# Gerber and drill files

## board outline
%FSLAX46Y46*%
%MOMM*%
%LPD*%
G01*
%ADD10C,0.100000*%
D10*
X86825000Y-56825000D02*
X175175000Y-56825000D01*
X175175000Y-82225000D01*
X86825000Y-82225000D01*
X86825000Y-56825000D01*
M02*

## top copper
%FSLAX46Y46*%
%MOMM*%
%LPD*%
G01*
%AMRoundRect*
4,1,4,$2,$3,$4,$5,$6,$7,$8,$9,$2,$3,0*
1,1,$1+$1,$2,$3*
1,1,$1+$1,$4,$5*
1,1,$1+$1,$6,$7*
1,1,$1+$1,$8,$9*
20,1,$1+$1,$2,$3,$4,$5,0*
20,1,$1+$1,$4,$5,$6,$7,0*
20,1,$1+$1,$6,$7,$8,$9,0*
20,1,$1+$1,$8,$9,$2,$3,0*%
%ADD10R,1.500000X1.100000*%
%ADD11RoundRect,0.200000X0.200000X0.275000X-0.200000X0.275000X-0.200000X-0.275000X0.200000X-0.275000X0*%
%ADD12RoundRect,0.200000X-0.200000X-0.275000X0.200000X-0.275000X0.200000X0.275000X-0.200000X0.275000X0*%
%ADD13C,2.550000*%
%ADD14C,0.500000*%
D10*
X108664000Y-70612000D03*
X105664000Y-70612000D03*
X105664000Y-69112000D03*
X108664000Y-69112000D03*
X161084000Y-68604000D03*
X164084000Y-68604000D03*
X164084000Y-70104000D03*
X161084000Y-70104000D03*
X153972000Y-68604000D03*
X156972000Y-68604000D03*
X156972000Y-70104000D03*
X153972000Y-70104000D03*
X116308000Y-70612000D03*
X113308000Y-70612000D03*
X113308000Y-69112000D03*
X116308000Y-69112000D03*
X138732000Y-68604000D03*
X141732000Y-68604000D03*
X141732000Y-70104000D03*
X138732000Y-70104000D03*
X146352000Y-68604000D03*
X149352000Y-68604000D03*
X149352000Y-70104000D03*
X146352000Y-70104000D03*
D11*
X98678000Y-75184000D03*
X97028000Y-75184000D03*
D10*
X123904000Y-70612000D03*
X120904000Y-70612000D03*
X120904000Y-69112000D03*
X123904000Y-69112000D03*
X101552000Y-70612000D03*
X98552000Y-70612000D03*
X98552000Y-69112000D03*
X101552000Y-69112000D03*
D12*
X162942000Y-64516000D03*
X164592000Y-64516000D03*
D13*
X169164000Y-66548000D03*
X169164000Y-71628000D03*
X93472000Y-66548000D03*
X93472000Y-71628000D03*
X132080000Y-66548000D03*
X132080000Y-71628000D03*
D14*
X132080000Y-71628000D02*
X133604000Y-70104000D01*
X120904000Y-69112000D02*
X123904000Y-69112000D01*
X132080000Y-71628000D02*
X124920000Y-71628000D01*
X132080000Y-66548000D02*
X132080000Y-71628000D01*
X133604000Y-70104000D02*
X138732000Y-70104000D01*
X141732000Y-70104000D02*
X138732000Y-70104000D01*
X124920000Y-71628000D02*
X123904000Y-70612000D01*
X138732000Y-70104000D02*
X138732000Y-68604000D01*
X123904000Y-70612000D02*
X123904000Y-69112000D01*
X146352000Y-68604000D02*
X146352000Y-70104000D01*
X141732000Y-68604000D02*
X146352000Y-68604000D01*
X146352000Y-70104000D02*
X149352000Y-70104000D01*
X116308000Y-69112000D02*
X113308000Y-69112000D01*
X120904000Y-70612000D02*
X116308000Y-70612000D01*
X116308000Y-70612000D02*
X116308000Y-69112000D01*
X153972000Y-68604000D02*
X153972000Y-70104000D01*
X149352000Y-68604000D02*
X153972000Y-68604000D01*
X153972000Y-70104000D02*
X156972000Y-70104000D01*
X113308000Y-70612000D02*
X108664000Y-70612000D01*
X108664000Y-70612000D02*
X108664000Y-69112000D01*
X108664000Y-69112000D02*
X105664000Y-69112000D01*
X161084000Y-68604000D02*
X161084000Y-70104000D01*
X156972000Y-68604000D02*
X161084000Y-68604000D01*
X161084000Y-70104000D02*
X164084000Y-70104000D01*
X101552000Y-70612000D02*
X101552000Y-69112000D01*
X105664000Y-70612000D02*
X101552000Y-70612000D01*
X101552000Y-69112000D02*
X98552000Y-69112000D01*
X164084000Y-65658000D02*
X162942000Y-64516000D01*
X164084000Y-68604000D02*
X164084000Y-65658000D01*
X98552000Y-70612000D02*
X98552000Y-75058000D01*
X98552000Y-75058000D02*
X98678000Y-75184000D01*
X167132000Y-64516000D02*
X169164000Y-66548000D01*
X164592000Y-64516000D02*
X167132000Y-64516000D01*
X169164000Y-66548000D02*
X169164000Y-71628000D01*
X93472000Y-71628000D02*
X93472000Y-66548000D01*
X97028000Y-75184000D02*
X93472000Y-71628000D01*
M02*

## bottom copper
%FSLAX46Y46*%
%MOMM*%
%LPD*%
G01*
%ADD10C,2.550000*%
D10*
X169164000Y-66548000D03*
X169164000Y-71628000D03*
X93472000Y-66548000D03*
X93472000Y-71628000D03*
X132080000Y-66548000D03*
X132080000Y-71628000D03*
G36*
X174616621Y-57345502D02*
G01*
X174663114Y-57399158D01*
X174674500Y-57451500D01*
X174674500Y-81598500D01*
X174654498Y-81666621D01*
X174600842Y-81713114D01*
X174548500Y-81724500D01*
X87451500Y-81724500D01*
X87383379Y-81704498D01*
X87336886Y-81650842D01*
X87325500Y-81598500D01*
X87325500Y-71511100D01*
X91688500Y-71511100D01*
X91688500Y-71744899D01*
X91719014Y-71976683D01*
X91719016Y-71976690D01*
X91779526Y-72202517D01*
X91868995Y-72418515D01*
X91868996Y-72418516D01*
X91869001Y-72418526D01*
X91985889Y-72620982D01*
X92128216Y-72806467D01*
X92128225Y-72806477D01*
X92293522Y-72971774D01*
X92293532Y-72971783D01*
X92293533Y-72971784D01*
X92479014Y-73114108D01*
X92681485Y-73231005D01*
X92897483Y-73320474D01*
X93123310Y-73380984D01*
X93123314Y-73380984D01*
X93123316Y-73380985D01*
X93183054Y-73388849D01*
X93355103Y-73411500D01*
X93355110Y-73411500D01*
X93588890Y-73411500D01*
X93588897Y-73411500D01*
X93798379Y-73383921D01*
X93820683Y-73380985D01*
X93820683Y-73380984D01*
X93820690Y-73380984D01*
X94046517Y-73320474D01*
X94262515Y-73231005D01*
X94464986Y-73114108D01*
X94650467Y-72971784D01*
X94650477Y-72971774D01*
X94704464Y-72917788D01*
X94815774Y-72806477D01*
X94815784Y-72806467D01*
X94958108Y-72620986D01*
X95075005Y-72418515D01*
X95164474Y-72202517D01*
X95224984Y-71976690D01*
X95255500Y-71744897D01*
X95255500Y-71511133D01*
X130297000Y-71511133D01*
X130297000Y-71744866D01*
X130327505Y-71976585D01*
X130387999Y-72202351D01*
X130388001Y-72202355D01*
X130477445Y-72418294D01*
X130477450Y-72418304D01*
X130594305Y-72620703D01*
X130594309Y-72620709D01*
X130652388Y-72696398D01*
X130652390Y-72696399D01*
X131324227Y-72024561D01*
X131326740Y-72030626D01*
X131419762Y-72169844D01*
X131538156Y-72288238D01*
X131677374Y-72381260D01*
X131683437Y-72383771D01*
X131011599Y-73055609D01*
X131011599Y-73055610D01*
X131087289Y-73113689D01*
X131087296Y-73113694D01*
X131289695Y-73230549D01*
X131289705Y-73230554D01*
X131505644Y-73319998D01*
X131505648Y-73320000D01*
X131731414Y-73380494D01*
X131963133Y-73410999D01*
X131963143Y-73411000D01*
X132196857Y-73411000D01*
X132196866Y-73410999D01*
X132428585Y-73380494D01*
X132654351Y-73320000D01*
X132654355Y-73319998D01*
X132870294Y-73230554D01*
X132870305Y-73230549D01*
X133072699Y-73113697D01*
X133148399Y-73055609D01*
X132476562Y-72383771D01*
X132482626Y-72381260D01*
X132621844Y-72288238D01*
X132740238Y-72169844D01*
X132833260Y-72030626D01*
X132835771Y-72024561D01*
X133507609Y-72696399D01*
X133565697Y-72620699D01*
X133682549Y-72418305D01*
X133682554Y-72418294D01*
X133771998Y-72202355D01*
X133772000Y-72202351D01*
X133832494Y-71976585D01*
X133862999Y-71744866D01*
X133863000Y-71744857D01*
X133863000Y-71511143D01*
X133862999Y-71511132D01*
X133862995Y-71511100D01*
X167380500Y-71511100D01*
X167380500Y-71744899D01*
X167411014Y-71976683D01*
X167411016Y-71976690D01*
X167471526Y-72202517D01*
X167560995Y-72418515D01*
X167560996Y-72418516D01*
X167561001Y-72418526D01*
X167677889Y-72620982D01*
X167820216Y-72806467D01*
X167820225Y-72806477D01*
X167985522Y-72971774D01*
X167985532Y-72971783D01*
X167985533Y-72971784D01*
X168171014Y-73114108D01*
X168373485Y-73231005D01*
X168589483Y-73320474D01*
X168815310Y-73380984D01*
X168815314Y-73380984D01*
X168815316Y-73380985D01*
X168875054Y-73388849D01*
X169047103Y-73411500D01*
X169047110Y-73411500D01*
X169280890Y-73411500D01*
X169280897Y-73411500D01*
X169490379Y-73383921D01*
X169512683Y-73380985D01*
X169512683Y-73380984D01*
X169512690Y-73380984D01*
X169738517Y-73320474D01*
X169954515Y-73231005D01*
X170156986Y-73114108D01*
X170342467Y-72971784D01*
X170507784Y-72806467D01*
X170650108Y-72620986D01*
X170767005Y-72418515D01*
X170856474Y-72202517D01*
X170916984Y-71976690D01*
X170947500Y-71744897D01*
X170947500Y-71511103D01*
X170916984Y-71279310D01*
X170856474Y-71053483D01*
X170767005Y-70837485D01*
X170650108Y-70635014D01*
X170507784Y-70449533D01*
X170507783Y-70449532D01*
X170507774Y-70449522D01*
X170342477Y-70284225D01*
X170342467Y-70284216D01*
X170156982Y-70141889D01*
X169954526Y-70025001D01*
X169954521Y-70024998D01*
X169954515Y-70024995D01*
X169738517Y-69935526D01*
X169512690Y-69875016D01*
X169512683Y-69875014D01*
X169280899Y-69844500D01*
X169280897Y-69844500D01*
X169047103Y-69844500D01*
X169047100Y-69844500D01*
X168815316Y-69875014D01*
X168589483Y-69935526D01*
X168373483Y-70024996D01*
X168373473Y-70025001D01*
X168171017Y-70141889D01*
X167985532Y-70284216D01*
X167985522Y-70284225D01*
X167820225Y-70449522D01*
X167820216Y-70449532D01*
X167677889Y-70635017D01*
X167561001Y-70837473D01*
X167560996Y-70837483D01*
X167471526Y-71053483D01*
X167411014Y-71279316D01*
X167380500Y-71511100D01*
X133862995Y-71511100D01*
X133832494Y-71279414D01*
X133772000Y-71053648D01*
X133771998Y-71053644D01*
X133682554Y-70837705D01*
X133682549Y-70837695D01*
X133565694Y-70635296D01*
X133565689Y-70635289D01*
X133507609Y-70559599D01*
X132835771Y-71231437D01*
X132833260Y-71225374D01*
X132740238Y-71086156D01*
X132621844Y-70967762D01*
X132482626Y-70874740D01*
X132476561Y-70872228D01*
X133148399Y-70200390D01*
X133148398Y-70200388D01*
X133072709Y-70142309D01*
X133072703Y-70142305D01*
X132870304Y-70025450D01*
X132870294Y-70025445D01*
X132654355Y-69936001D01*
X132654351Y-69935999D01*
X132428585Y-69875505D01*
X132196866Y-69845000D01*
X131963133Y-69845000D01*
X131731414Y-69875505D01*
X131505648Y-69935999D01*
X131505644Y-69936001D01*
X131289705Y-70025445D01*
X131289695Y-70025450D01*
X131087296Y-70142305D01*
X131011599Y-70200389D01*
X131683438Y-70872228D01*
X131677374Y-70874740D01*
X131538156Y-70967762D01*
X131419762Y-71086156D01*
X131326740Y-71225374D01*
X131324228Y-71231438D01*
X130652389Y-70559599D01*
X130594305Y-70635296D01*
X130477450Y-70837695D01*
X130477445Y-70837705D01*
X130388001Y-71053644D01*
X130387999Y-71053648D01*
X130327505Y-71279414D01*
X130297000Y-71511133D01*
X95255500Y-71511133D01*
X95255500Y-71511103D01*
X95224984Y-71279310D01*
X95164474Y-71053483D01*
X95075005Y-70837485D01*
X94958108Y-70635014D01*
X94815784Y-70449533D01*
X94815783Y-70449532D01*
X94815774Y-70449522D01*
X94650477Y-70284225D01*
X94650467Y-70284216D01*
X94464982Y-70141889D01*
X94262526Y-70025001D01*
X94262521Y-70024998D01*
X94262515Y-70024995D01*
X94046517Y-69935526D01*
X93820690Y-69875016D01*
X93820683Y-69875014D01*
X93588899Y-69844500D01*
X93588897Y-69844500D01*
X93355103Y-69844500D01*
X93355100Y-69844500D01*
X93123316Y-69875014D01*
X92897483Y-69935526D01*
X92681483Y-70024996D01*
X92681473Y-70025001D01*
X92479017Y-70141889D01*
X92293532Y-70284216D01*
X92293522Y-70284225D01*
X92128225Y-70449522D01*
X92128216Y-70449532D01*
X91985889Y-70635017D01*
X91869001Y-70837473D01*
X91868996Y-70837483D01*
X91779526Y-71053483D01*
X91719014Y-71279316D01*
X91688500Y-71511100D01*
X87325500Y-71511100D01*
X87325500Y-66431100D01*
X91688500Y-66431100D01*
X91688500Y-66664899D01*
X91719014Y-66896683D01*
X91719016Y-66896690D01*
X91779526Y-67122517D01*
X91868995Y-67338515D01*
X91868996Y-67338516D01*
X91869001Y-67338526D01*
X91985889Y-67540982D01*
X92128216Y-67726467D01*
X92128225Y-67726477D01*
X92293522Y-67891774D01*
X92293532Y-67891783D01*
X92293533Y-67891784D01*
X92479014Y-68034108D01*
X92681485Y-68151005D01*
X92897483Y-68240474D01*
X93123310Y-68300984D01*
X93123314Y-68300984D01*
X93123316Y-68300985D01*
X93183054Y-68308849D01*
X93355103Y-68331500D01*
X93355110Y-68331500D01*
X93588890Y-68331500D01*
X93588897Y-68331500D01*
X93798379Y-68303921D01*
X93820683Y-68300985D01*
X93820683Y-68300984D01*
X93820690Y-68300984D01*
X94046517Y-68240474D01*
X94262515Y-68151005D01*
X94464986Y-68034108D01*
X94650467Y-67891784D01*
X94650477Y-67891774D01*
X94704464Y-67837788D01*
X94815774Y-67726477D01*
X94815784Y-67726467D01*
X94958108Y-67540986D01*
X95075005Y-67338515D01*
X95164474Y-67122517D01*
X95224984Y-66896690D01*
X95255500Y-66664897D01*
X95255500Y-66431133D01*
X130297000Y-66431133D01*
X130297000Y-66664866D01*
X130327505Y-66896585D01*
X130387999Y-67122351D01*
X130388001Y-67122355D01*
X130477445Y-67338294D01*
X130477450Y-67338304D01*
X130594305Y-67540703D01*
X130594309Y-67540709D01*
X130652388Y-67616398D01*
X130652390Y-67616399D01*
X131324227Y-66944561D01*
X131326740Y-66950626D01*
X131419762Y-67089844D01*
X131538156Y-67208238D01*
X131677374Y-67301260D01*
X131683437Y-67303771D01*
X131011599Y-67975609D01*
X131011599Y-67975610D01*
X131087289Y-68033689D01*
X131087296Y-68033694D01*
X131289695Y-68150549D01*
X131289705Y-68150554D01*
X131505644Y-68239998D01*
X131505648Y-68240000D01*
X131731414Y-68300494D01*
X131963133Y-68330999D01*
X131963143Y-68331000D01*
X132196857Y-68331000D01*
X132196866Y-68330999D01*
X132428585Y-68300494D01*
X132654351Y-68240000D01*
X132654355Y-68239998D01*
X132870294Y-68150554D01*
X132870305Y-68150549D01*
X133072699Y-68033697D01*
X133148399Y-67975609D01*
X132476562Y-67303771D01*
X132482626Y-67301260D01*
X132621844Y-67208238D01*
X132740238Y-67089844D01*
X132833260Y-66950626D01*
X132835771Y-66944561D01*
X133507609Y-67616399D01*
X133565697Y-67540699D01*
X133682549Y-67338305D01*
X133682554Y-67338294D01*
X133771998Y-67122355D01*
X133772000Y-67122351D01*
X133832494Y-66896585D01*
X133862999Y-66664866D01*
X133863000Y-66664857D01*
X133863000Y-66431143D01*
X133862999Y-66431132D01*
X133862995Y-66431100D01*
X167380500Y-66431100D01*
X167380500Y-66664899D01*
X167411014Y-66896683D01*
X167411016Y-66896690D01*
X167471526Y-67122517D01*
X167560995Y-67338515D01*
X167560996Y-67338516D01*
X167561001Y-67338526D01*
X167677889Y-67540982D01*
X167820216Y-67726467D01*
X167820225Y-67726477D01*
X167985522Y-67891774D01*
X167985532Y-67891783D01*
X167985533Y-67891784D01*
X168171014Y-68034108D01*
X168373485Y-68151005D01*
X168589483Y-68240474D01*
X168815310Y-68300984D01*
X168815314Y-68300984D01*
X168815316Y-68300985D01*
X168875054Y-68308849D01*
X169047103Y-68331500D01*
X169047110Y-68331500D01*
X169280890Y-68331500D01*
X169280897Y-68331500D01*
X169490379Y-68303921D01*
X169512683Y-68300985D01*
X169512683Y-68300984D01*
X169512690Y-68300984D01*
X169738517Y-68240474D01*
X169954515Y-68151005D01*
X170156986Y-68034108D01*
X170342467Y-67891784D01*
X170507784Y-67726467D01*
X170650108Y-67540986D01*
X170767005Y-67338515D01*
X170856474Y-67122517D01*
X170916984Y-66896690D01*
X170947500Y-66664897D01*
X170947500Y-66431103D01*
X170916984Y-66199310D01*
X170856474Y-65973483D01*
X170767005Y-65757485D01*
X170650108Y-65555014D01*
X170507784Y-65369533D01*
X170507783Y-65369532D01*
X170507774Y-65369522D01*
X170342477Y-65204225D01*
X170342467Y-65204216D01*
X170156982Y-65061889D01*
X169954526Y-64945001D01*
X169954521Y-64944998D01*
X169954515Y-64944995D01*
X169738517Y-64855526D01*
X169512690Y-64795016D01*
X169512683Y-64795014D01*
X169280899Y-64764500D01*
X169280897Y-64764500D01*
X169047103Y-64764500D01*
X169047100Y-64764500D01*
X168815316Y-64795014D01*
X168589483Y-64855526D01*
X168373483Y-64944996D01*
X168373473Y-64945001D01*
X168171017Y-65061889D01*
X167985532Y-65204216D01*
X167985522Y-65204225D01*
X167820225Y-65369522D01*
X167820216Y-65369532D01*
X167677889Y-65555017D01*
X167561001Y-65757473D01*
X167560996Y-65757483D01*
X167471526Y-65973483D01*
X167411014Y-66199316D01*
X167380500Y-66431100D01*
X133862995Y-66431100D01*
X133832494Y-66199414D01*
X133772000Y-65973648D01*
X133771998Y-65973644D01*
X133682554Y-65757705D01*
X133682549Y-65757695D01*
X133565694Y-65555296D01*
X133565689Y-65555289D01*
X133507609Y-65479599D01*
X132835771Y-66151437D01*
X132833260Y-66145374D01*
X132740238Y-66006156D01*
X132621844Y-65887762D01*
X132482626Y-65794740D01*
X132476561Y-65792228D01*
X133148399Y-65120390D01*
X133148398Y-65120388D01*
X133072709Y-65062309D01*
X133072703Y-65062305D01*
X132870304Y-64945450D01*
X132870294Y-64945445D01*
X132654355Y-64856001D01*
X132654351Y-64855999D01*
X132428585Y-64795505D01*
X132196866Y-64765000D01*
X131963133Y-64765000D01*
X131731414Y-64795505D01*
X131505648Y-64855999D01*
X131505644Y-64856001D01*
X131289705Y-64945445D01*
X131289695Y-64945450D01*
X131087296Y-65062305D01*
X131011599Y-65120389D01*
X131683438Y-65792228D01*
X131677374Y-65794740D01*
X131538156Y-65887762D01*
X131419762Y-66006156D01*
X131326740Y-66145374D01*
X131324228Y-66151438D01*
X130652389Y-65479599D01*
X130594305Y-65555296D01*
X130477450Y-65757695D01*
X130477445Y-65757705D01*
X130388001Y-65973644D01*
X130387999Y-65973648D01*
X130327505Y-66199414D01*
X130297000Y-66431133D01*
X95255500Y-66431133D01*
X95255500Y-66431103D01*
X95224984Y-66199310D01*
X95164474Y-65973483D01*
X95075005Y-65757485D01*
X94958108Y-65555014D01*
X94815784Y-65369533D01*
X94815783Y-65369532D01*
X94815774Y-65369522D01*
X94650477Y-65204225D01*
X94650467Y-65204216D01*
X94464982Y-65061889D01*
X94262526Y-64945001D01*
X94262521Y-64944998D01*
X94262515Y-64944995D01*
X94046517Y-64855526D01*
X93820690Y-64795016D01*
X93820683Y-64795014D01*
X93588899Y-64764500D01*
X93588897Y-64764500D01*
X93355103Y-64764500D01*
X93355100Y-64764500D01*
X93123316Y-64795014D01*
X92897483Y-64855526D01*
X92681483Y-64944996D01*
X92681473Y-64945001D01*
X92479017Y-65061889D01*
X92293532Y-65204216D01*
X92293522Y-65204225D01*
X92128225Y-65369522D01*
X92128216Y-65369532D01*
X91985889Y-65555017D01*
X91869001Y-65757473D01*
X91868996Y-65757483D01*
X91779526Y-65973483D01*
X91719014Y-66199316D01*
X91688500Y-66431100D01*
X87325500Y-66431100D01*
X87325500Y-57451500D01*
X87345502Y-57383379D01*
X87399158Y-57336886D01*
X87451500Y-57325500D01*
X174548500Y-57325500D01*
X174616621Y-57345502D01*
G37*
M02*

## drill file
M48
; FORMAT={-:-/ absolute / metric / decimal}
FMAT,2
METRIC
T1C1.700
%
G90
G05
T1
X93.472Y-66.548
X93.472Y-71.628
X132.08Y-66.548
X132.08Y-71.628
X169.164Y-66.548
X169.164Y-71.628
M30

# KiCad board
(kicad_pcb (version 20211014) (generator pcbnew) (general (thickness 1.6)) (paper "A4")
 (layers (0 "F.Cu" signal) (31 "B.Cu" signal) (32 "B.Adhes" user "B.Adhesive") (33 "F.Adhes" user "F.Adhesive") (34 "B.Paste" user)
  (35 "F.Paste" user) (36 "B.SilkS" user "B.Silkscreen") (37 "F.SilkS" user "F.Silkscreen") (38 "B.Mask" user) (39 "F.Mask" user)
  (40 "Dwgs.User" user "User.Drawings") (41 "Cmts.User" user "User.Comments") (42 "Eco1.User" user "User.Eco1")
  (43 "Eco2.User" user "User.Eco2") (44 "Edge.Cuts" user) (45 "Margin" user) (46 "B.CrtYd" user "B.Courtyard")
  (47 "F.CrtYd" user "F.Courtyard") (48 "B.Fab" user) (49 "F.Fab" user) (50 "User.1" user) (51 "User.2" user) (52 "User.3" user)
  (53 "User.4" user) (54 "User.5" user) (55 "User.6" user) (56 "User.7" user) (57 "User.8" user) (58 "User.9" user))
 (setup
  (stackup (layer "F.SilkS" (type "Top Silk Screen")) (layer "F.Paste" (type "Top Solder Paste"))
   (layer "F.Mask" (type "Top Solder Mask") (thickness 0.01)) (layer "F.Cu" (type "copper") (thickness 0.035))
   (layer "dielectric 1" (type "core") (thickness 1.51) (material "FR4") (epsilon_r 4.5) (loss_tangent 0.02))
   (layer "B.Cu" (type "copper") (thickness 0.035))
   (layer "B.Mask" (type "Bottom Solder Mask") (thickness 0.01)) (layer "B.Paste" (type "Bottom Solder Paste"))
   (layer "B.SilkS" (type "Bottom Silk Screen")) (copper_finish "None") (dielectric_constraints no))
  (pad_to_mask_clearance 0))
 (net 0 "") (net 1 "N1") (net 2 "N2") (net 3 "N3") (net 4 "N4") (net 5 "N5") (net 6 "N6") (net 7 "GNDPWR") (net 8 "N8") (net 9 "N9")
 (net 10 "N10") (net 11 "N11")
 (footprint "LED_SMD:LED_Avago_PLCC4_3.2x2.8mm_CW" (layer "F.Cu") (at 107.164 69.862 180)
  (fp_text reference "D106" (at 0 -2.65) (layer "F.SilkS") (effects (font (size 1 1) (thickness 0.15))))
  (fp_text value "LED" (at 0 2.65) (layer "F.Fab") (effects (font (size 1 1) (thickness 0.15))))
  (pad "1" smd rect (at -1.5 -0.75 180) (size 1.5 1.1) (layers "F.Cu" "F.Paste" "F.Mask") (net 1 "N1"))
  (pad "2" smd rect (at 1.5 -0.75 180) (size 1.5 1.1) (layers "F.Cu" "F.Paste" "F.Mask") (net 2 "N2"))
  (pad "3" smd rect (at 1.5 0.75 180) (size 1.5 1.1) (layers "F.Cu" "F.Paste" "F.Mask") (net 1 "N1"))
  (pad "4" smd rect (at -1.5 0.75 180) (size 1.5 1.1) (layers "F.Cu" "F.Paste" "F.Mask") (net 1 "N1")))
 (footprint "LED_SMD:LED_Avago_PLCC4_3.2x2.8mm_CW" (layer "F.Cu") (at 162.584 69.354)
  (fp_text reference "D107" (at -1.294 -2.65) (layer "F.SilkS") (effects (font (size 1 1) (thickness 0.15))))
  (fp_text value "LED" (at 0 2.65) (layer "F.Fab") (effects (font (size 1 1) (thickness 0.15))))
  (pad "1" smd rect (at -1.5 -0.75) (size 1.5 1.1) (layers "F.Cu" "F.Paste" "F.Mask") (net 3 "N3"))
  (pad "2" smd rect (at 1.5 -0.75) (size 1.5 1.1) (layers "F.Cu" "F.Paste" "F.Mask") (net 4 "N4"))
  (pad "3" smd rect (at 1.5 0.75) (size 1.5 1.1) (layers "F.Cu" "F.Paste" "F.Mask") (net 3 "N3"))
  (pad "4" smd rect (at -1.5 0.75) (size 1.5 1.1) (layers "F.Cu" "F.Paste" "F.Mask") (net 3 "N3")))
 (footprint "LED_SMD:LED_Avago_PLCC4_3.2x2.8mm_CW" (layer "F.Cu") (at 155.472 69.354)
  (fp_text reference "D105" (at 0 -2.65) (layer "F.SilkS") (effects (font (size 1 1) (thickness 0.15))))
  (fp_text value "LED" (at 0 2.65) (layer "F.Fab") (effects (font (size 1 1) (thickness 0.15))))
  (pad "1" smd rect (at -1.5 -0.75) (size 1.5 1.1) (layers "F.Cu" "F.Paste" "F.Mask") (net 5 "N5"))
  (pad "2" smd rect (at 1.5 -0.75) (size 1.5 1.1) (layers "F.Cu" "F.Paste" "F.Mask") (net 3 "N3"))
  (pad "3" smd rect (at 1.5 0.75) (size 1.5 1.1) (layers "F.Cu" "F.Paste" "F.Mask") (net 5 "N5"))
  (pad "4" smd rect (at -1.5 0.75) (size 1.5 1.1) (layers "F.Cu" "F.Paste" "F.Mask") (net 5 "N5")))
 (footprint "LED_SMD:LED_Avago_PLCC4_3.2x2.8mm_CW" (layer "F.Cu") (at 114.808 69.862 180)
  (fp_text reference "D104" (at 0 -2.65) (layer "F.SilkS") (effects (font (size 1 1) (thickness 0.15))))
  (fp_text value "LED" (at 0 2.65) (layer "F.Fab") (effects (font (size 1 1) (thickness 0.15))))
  (pad "1" smd rect (at -1.5 -0.75 180) (size 1.5 1.1) (layers "F.Cu" "F.Paste" "F.Mask") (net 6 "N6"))
  (pad "2" smd rect (at 1.5 -0.75 180) (size 1.5 1.1) (layers "F.Cu" "F.Paste" "F.Mask") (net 1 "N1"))
  (pad "3" smd rect (at 1.5 0.75 180) (size 1.5 1.1) (layers "F.Cu" "F.Paste" "F.Mask") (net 6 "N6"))
  (pad "4" smd rect (at -1.5 0.75 180) (size 1.5 1.1) (layers "F.Cu" "F.Paste" "F.Mask") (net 6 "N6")))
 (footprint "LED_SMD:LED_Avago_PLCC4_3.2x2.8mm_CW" (layer "F.Cu") (at 140.232 69.354)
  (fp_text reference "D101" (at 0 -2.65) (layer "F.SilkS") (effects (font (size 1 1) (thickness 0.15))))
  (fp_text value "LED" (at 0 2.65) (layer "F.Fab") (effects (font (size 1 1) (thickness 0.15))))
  (pad "1" smd rect (at -1.5 -0.75) (size 1.5 1.1) (layers "F.Cu" "F.Paste" "F.Mask") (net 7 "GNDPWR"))
  (pad "2" smd rect (at 1.5 -0.75) (size 1.5 1.1) (layers "F.Cu" "F.Paste" "F.Mask") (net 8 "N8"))
  (pad "3" smd rect (at 1.5 0.75) (size 1.5 1.1) (layers "F.Cu" "F.Paste" "F.Mask") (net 7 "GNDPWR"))
  (pad "4" smd rect (at -1.5 0.75) (size 1.5 1.1) (layers "F.Cu" "F.Paste" "F.Mask") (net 7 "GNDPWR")))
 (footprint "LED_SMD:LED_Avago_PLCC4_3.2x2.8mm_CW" (layer "F.Cu") (at 147.852 69.354)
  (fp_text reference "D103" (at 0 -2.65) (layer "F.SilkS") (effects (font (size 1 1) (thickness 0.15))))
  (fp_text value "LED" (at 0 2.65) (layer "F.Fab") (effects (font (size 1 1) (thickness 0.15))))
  (pad "1" smd rect (at -1.5 -0.75) (size 1.5 1.1) (layers "F.Cu" "F.Paste" "F.Mask") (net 8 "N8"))
  (pad "2" smd rect (at 1.5 -0.75) (size 1.5 1.1) (layers "F.Cu" "F.Paste" "F.Mask") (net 5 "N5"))
  (pad "3" smd rect (at 1.5 0.75) (size 1.5 1.1) (layers "F.Cu" "F.Paste" "F.Mask") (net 8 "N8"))
  (pad "4" smd rect (at -1.5 0.75) (size 1.5 1.1) (layers "F.Cu" "F.Paste" "F.Mask") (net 8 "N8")))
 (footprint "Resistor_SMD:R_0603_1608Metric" (layer "F.Cu") (at 97.853 75.184 180)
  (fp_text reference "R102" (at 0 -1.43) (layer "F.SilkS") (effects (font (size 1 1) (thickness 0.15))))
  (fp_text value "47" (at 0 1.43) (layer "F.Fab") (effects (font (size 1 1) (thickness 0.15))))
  (pad "1" smd roundrect (at -0.825 0 180) (size 0.8 0.95) (layers "F.Cu" "F.Paste" "F.Mask") (roundrect_rratio 0.25) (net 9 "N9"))
  (pad "2" smd roundrect (at 0.825 0 180) (size 0.8 0.95) (layers "F.Cu" "F.Paste" "F.Mask") (roundrect_rratio 0.25) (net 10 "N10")))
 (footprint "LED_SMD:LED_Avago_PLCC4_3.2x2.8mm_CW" (layer "F.Cu") (at 122.404 69.862 180)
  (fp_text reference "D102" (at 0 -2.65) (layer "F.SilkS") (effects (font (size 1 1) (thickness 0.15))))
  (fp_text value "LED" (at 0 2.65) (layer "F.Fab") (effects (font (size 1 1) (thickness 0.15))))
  (pad "1" smd rect (at -1.5 -0.75 180) (size 1.5 1.1) (layers "F.Cu" "F.Paste" "F.Mask") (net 7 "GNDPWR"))
  (pad "2" smd rect (at 1.5 -0.75 180) (size 1.5 1.1) (layers "F.Cu" "F.Paste" "F.Mask") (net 6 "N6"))
  (pad "3" smd rect (at 1.5 0.75 180) (size 1.5 1.1) (layers "F.Cu" "F.Paste" "F.Mask") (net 7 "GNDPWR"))
  (pad "4" smd rect (at -1.5 0.75 180) (size 1.5 1.1) (layers "F.Cu" "F.Paste" "F.Mask") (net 7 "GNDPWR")))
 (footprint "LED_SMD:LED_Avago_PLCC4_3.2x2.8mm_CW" (layer "F.Cu") (at 100.052 69.862 180)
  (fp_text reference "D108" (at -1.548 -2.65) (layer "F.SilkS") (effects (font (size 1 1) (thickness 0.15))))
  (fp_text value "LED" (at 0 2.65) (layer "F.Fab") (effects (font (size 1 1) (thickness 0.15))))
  (pad "1" smd rect (at -1.5 -0.75 180) (size 1.5 1.1) (layers "F.Cu" "F.Paste" "F.Mask") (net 2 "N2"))
  (pad "2" smd rect (at 1.5 -0.75 180) (size 1.5 1.1) (layers "F.Cu" "F.Paste" "F.Mask") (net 9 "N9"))
  (pad "3" smd rect (at 1.5 0.75 180) (size 1.5 1.1) (layers "F.Cu" "F.Paste" "F.Mask") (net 2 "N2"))
  (pad "4" smd rect (at -1.5 0.75 180) (size 1.5 1.1) (layers "F.Cu" "F.Paste" "F.Mask") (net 2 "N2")))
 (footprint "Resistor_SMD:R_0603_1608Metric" (layer "F.Cu") (at 163.767 64.516)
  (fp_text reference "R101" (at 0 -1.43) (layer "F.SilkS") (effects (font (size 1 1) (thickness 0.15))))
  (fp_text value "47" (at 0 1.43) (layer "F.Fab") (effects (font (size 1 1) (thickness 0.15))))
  (pad "1" smd roundrect (at -0.825 0) (size 0.8 0.95) (layers "F.Cu" "F.Paste" "F.Mask") (roundrect_rratio 0.25) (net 4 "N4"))
  (pad "2" smd roundrect (at 0.825 0) (size 0.8 0.95) (layers "F.Cu" "F.Paste" "F.Mask") (roundrect_rratio 0.25) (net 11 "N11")))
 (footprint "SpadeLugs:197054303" (layer "B.Cu") (at 169.164 66.548 -90)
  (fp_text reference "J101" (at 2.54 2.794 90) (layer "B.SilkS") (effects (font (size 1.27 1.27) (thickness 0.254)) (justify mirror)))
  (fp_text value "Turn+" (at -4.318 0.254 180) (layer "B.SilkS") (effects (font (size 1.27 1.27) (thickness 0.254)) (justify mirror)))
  (pad "1" thru_hole circle locked (at 0 0 270) (size 2.55 2.55) (drill 1.7) (layers *.Cu *.Mask) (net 11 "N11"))
  (pad "2" thru_hole circle locked (at 5.08 0 270) (size 2.55 2.55) (drill 1.7) (layers *.Cu *.Mask) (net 11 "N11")))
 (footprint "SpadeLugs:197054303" (layer "B.Cu") (at 93.472 66.548 -90)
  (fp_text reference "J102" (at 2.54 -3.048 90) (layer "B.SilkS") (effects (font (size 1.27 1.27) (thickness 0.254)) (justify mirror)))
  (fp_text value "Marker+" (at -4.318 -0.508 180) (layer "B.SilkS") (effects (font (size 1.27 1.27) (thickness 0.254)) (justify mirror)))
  (pad "1" thru_hole circle locked (at 0 0 270) (size 2.55 2.55) (drill 1.7) (layers *.Cu *.Mask) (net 10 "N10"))
  (pad "2" thru_hole circle locked (at 5.08 0 270) (size 2.55 2.55) (drill 1.7) (layers *.Cu *.Mask) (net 10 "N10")))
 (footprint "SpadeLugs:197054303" (layer "B.Cu") (at 132.08 66.548 -90)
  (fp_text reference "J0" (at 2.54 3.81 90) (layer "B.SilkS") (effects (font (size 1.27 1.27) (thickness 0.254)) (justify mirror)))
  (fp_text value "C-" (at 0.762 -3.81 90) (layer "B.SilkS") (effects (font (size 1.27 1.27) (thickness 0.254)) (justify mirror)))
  (pad "1" thru_hole circle locked (at 0 0 270) (size 2.55 2.55) (drill 1.7) (layers *.Cu *.Mask) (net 7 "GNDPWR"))
  (pad "2" thru_hole circle locked (at 5.08 0 270) (size 2.55 2.55) (drill 1.7) (layers *.Cu *.Mask) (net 7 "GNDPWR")))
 (gr_rect (start 86.825 56.825) (end 175.175 82.225) (layer "Edge.Cuts") (width 0.1) (fill none))
 (segment (start 132.08 71.628) (end 133.604 70.104) (width 0.5) (layer "F.Cu") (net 7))
 (segment (start 120.904 69.112) (end 123.904 69.112) (width 0.5) (layer "F.Cu") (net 7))
 (segment (start 132.08 71.628) (end 124.92 71.628) (width 0.5) (layer "F.Cu") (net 7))
 (segment (start 132.08 66.548) (end 132.08 71.628) (width 0.5) (layer "F.Cu") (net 7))
 (segment (start 133.604 70.104) (end 138.732 70.104) (width 0.5) (layer "F.Cu") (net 7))
 (segment (start 141.732 70.104) (end 138.732 70.104) (width 0.5) (layer "F.Cu") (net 7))
 (segment (start 124.92 71.628) (end 123.904 70.612) (width 0.5) (layer "F.Cu") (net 7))
 (segment (start 138.732 70.104) (end 138.732 68.604) (width 0.5) (layer "F.Cu") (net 7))
 (segment (start 123.904 70.612) (end 123.904 69.112) (width 0.5) (layer "F.Cu") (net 7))
 (segment (start 146.352 68.604) (end 146.352 70.104) (width 0.5) (layer "F.Cu") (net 8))
 (segment (start 141.732 68.604) (end 146.352 68.604) (width 0.5) (layer "F.Cu") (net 8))
 (segment (start 146.352 70.104) (end 149.352 70.104) (width 0.5) (layer "F.Cu") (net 8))
 (segment (start 116.308 69.112) (end 113.308 69.112) (width 0.5) (layer "F.Cu") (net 6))
 (segment (start 120.904 70.612) (end 116.308 70.612) (width 0.5) (layer "F.Cu") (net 6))
 (segment (start 116.308 70.612) (end 116.308 69.112) (width 0.5) (layer "F.Cu") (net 6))
 (segment (start 153.972 68.604) (end 153.972 70.104) (width 0.5) (layer "F.Cu") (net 5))
 (segment (start 149.352 68.604) (end 153.972 68.604) (width 0.5) (layer "F.Cu") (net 5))
 (segment (start 153.972 70.104) (end 156.972 70.104) (width 0.5) (layer "F.Cu") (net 5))
 (segment (start 113.308 70.612) (end 108.664 70.612) (width 0.5) (layer "F.Cu") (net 1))
 (segment (start 108.664 70.612) (end 108.664 69.112) (width 0.5) (layer "F.Cu") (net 1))
 (segment (start 108.664 69.112) (end 105.664 69.112) (width 0.5) (layer "F.Cu") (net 1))
 (segment (start 161.084 68.604) (end 161.084 70.104) (width 0.5) (layer "F.Cu") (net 3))
 (segment (start 156.972 68.604) (end 161.084 68.604) (width 0.5) (layer "F.Cu") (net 3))
 (segment (start 161.084 70.104) (end 164.084 70.104) (width 0.5) (layer "F.Cu") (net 3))
 (segment (start 101.552 70.612) (end 101.552 69.112) (width 0.5) (layer "F.Cu") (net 2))
 (segment (start 105.664 70.612) (end 101.552 70.612) (width 0.5) (layer "F.Cu") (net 2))
 (segment (start 101.552 69.112) (end 98.552 69.112) (width 0.5) (layer "F.Cu") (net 2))
 (segment (start 164.084 65.658) (end 162.942 64.516) (width 0.5) (layer "F.Cu") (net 4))
 (segment (start 164.084 68.604) (end 164.084 65.658) (width 0.5) (layer "F.Cu") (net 4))
 (segment (start 98.552 70.612) (end 98.552 75.058) (width 0.5) (layer "F.Cu") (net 9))
 (segment (start 98.552 75.058) (end 98.678 75.184) (width 0.5) (layer "F.Cu") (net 9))
 (segment (start 167.132 64.516) (end 169.164 66.548) (width 0.5) (layer "F.Cu") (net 11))
 (segment (start 164.592 64.516) (end 167.132 64.516) (width 0.5) (layer "F.Cu") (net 11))
 (segment (start 169.164 66.548) (end 169.164 71.628) (width 0.5) (layer "F.Cu") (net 11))
 (segment (start 93.472 71.628) (end 93.472 66.548) (width 0.5) (layer "F.Cu") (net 10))
 (segment (start 97.028 75.184) (end 93.472 71.628) (width 0.5) (layer "F.Cu") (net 10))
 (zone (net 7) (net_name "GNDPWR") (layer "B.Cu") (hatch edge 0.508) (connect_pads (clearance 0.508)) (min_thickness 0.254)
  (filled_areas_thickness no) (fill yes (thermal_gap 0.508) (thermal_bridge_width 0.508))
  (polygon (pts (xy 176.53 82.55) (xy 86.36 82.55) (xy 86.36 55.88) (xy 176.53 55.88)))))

